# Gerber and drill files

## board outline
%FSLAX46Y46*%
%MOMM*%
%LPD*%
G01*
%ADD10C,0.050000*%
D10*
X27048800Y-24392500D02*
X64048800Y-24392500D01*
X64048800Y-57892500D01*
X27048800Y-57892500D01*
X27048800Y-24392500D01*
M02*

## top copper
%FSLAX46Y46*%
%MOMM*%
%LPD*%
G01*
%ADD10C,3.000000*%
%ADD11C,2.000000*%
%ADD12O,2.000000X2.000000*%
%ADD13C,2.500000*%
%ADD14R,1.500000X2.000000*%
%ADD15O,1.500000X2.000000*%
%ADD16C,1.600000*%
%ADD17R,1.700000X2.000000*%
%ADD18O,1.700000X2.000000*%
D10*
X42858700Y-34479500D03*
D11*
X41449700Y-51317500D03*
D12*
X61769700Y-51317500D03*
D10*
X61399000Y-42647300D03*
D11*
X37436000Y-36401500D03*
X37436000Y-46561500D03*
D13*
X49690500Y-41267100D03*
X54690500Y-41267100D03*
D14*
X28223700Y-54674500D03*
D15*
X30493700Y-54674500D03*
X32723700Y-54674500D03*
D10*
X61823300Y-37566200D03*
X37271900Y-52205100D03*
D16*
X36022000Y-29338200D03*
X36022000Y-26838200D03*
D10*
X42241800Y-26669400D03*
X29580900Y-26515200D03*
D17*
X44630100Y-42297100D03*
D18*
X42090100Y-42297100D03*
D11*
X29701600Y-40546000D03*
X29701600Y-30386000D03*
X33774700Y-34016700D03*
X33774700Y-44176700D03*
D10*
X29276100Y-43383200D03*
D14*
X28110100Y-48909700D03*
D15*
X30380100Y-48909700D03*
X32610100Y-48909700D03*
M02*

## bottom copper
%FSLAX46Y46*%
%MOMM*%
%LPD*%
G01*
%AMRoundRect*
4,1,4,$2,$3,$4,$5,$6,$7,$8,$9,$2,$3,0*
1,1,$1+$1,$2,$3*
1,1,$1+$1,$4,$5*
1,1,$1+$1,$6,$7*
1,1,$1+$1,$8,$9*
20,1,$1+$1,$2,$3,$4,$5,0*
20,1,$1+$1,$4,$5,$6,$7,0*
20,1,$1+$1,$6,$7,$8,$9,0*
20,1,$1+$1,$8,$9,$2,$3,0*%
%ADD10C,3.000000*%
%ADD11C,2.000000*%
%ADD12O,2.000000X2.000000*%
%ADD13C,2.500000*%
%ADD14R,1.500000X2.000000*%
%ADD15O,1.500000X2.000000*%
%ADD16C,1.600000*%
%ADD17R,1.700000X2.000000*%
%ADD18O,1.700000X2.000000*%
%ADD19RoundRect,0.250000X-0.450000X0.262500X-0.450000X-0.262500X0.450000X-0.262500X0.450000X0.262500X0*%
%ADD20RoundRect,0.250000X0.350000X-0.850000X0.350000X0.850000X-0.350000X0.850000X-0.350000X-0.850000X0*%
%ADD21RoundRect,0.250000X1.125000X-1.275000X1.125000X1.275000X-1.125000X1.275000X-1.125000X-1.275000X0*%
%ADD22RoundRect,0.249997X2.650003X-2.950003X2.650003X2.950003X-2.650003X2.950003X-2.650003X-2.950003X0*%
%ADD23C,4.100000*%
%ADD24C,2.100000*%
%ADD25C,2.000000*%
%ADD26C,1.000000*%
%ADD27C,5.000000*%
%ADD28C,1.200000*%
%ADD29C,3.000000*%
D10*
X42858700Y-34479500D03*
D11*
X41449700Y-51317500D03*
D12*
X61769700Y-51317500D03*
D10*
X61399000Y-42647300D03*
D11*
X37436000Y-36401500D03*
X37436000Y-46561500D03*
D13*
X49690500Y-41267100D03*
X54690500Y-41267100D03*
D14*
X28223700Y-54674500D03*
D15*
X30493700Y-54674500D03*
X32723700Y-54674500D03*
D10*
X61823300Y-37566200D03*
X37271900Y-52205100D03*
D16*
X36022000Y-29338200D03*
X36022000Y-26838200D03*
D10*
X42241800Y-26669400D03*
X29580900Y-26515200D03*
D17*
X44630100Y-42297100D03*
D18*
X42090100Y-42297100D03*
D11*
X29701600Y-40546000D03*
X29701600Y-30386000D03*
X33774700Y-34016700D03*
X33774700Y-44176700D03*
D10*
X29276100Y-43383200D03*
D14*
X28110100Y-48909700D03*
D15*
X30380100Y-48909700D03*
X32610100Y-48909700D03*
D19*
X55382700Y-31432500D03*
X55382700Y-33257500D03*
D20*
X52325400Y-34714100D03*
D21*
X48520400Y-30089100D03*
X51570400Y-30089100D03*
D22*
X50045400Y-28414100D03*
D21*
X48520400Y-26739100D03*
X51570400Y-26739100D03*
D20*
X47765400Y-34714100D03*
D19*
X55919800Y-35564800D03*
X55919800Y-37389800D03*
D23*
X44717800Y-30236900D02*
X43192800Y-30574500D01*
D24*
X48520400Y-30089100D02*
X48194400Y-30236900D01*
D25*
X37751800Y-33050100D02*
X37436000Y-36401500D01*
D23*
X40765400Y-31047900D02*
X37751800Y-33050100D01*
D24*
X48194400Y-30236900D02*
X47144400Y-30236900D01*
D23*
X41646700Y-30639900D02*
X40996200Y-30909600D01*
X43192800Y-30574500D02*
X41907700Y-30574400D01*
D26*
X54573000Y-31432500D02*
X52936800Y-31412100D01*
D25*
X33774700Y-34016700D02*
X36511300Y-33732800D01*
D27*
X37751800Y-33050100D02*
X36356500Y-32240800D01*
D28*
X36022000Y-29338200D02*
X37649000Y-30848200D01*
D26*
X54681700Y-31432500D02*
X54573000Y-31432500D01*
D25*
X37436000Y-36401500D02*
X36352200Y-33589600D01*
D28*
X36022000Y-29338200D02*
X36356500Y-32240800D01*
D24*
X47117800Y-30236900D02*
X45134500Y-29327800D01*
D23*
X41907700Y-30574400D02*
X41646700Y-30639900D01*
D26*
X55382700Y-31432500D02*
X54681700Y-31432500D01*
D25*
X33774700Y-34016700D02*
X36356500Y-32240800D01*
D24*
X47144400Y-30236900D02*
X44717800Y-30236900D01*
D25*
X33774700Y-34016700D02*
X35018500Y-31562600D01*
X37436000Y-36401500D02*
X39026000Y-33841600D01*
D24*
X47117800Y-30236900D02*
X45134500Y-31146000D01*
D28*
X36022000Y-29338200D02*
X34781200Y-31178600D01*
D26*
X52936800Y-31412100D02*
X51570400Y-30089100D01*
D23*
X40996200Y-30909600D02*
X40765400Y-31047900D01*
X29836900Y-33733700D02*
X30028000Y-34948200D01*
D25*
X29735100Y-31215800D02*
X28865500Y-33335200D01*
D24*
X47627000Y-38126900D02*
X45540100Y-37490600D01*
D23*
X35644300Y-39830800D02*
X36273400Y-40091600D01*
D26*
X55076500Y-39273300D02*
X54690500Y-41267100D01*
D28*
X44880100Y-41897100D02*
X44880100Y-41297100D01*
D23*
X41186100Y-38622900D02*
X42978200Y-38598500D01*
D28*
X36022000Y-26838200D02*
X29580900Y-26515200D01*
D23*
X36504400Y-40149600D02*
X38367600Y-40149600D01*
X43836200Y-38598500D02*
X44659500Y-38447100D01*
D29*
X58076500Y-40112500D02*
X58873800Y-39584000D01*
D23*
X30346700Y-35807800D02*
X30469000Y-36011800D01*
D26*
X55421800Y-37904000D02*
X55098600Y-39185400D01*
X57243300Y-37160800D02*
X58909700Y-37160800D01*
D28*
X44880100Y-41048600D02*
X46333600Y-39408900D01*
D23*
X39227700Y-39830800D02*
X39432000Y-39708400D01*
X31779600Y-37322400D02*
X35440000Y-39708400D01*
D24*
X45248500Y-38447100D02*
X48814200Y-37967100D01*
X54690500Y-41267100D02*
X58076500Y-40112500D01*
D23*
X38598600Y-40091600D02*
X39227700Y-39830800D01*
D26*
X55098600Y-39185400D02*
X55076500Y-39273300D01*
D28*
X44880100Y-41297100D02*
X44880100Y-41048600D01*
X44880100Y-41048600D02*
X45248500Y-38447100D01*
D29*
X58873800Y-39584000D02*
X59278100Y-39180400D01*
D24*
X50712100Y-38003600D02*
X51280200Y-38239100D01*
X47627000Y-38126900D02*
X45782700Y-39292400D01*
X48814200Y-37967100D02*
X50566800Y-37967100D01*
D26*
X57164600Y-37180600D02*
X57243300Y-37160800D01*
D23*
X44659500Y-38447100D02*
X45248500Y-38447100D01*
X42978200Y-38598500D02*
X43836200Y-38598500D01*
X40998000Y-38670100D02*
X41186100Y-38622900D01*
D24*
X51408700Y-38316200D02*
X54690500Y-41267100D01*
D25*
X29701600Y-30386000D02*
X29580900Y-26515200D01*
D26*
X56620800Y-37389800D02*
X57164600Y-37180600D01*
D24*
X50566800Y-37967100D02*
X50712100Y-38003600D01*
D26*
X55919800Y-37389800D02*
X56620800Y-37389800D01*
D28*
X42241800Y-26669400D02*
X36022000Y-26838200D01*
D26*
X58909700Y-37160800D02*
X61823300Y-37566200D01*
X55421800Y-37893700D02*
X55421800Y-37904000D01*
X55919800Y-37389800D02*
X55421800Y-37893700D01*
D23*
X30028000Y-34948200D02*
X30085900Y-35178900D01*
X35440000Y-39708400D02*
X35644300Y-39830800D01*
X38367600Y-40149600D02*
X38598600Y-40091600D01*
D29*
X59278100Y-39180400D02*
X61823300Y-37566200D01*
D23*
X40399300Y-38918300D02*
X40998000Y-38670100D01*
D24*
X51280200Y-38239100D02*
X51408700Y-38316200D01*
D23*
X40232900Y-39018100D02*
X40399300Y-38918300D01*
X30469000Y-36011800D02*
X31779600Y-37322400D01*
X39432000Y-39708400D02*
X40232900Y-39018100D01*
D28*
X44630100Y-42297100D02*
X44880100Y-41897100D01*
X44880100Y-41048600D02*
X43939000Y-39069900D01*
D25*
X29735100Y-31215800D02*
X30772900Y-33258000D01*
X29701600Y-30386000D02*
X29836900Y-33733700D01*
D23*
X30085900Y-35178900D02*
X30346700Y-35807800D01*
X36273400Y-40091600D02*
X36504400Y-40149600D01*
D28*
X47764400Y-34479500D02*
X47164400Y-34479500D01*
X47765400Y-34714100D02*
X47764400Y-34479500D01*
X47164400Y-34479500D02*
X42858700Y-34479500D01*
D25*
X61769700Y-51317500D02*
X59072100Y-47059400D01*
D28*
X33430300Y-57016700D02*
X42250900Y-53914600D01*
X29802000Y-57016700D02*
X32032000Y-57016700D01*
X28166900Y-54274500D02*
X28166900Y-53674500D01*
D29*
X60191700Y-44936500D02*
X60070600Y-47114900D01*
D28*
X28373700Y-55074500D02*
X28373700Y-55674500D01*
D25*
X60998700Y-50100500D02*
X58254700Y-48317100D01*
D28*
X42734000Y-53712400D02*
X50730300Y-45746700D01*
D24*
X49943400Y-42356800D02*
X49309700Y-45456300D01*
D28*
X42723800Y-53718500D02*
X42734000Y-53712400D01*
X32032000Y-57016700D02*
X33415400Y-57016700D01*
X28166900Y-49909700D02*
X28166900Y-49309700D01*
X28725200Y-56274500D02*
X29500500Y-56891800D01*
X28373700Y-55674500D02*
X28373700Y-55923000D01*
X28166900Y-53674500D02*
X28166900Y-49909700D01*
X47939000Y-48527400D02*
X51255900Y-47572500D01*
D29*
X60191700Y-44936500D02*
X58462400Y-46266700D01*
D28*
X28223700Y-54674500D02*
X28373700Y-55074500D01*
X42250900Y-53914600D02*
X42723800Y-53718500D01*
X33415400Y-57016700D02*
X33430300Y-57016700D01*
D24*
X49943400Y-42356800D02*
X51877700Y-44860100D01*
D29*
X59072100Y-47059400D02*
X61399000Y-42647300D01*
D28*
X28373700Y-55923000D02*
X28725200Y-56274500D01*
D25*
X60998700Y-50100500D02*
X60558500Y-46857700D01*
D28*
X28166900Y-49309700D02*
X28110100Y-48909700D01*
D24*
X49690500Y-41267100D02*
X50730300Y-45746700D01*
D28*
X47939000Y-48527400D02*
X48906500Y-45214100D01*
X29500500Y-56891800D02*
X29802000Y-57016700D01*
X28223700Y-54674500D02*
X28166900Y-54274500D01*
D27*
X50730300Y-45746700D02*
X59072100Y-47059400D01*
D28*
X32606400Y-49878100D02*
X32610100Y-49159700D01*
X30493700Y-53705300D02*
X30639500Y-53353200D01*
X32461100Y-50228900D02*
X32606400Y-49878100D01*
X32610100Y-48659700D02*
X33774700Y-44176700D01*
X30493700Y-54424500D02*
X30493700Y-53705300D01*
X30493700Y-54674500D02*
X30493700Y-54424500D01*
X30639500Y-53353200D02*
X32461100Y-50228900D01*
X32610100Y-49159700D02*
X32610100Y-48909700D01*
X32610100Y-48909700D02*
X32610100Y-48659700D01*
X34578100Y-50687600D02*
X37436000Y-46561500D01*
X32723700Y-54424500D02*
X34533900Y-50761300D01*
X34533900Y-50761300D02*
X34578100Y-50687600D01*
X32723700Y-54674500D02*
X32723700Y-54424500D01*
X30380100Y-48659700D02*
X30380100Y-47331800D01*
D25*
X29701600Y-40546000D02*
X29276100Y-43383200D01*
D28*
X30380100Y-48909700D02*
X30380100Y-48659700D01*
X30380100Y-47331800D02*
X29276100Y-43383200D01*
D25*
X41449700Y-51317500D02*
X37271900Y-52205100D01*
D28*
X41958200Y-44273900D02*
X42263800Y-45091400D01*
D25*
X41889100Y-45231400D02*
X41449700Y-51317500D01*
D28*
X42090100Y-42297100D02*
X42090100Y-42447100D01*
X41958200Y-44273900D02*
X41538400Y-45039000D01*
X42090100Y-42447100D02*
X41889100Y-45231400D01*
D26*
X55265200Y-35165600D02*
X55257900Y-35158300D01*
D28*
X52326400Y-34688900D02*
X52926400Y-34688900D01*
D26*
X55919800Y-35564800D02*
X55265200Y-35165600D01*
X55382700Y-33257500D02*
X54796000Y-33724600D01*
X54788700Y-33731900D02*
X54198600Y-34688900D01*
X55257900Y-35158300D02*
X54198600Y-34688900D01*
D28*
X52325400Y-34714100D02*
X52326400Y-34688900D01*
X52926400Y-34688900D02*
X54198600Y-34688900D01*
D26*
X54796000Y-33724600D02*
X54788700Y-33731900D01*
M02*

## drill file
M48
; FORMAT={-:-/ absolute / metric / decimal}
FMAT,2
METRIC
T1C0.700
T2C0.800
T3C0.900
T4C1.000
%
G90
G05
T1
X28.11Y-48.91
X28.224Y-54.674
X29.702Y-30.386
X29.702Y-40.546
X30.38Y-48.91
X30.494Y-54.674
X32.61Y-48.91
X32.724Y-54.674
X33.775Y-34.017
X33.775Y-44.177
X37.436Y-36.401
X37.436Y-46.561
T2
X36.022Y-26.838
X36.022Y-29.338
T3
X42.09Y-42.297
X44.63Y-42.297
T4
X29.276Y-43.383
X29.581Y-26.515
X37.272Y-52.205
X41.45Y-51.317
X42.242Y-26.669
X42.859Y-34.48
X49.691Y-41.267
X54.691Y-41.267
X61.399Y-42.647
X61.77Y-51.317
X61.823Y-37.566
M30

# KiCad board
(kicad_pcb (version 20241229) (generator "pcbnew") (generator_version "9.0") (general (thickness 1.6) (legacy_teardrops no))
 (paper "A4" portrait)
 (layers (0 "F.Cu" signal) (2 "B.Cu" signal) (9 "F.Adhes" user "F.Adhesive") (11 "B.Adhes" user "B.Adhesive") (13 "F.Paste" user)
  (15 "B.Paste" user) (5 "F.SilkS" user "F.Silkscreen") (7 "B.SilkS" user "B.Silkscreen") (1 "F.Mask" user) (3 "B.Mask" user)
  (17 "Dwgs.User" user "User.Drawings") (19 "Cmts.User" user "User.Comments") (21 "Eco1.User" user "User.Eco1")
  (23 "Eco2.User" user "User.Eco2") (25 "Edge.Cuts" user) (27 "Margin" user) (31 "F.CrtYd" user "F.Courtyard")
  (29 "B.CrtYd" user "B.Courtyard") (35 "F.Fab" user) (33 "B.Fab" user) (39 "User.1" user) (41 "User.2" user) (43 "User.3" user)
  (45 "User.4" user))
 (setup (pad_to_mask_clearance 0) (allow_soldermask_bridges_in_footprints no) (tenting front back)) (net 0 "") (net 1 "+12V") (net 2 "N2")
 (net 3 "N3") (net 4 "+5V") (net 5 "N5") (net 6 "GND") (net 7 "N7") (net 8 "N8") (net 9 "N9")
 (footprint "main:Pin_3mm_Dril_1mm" (layer "F.Cu") (at 42.8587 34.4795)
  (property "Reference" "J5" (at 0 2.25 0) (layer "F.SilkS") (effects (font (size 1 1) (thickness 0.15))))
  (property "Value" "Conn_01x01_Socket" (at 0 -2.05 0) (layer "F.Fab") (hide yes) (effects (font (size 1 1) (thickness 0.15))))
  (pad "1" thru_hole circle (at 0 0) (size 3 3) (drill 1) (layers "*.Cu" "*.Mask") (remove_unused_layers no) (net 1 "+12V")))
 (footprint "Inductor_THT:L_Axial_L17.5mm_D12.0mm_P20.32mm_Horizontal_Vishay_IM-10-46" (layer "F.Cu") (at 41.4497 51.3175)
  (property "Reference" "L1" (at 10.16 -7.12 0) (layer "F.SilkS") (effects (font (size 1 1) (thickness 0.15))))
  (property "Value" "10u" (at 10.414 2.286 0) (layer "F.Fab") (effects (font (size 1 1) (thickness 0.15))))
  (pad "1" thru_hole circle (at 0 0) (size 2 2) (drill 1) (layers "*.Cu" "*.Mask") (remove_unused_layers no) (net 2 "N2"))
  (pad "2" thru_hole oval (at 20.32 0) (size 2 2) (drill 1) (layers "*.Cu" "*.Mask") (remove_unused_layers no) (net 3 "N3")))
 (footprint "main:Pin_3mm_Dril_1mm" (layer "F.Cu") (at 61.399 42.6473)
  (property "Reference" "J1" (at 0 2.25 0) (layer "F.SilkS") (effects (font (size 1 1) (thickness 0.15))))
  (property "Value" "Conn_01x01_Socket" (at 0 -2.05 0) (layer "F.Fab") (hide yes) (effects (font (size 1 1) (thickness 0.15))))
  (pad "1" thru_hole circle (at 0 0) (size 3 3) (drill 1) (layers "*.Cu" "*.Mask") (remove_unused_layers no) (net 3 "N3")))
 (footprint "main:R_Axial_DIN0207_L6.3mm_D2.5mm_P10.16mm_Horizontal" (layer "F.Cu") (at 37.436 36.4015 -90)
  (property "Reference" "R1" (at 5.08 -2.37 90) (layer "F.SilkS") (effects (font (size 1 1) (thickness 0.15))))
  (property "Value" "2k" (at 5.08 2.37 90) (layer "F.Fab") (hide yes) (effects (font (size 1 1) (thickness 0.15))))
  (pad "1" thru_hole circle (at 0 0 270) (size 2 2) (drill 0.7) (layers "*.Cu" "*.Mask") (remove_unused_layers no) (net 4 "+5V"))
  (pad "2" thru_hole circle (at 10.16 0 270) (size 2 2) (drill 0.7) (layers "*.Cu" "*.Mask") (remove_unused_layers no) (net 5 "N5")))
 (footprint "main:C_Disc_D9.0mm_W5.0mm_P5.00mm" (layer "F.Cu") (at 49.6905 41.2671)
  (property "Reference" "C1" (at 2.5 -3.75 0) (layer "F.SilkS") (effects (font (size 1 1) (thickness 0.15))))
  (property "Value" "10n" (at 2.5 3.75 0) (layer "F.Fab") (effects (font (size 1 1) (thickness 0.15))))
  (pad "1" thru_hole circle (at 0 0) (size 2.5 2.5) (drill 1) (layers "*.Cu" "*.Mask") (remove_unused_layers no) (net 3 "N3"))
  (pad "2" thru_hole circle (at 5 0) (size 2.5 2.5) (drill 1) (layers "*.Cu" "*.Mask") (remove_unused_layers no) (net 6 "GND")))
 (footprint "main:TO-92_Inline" (layer "F.Cu") (at 29.2237 54.6745)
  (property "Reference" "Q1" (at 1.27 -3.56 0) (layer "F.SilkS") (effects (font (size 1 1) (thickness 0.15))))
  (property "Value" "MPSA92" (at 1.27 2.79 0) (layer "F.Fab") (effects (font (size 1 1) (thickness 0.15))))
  (pad "1" thru_hole rect (at -1 0) (size 1.5 2) (drill 0.7) (layers "*.Cu" "*.Mask") (remove_unused_layers no) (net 3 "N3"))
  (pad "2" thru_hole oval (at 1.27 0) (size 1.5 2) (drill 0.7) (layers "*.Cu" "*.Mask") (remove_unused_layers no) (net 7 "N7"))
  (pad "3" thru_hole oval (at 3.5 0) (size 1.5 2) (drill 0.7) (layers "*.Cu" "*.Mask") (remove_unused_layers no) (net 5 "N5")))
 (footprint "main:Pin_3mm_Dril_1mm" (layer "F.Cu") (at 61.8233 37.5662)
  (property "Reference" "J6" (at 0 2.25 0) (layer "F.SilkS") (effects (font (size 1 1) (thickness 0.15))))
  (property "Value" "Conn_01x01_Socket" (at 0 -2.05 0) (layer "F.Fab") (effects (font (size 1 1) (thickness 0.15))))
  (pad "1" thru_hole circle (at 0 0) (size 3 3) (drill 1) (layers "*.Cu" "*.Mask") (remove_unused_layers no) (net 6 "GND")))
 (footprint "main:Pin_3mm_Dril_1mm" (layer "F.Cu") (at 37.2719 52.2051)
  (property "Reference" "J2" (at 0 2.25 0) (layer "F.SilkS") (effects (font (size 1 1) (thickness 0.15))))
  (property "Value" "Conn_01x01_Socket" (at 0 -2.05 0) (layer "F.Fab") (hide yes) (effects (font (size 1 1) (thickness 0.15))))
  (pad "1" thru_hole circle (at 0 0) (size 3 3) (drill 1) (layers "*.Cu" "*.Mask") (remove_unused_layers no) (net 2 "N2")))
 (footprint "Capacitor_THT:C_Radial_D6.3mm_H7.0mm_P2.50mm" (layer "F.Cu") (at 36.022 29.3382 90)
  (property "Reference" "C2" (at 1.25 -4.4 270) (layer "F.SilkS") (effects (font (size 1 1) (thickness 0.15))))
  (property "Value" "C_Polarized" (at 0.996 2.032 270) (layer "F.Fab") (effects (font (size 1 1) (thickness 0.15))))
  (pad "1" thru_hole circle (at 0 0 90) (size 1.6 1.6) (drill 0.8) (layers "*.Cu" "*.Mask") (remove_unused_layers no) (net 4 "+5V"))
  (pad "2" thru_hole circle (at 2.5 0 90) (size 1.6 1.6) (drill 0.8) (layers "*.Cu" "*.Mask") (remove_unused_layers no) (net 6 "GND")))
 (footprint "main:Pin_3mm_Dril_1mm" (layer "F.Cu") (at 42.2418 26.6694 -90)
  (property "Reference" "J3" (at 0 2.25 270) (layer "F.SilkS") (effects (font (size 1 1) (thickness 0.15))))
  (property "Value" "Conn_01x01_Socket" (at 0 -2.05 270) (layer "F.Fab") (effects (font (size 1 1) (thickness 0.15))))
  (pad "1" thru_hole circle (at 0 0 270) (size 3 3) (drill 1) (layers "*.Cu" "*.Mask") (remove_unused_layers no) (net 6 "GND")))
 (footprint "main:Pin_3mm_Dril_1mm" (layer "F.Cu") (at 29.5809 26.5152)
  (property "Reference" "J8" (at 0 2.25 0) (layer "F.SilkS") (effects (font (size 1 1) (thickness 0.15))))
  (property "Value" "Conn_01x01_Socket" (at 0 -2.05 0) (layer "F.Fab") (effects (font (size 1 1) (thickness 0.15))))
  (pad "1" thru_hole circle (at 0 0) (size 3 3) (drill 1) (layers "*.Cu" "*.Mask") (remove_unused_layers no) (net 6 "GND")))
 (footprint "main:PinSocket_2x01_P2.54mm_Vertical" (layer "F.Cu") (at 44.6301 42.2971)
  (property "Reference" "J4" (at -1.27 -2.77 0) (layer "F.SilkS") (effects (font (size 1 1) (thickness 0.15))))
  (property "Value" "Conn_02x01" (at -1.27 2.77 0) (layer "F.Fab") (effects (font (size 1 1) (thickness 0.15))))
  (pad "1" thru_hole rect (at 0 0) (size 1.7 2) (drill 0.9) (layers "*.Cu" "*.Mask") (remove_unused_layers no) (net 6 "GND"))
  (pad "2" thru_hole oval (at -2.54 0) (size 1.7 2) (drill 0.9) (layers "*.Cu" "*.Mask") (remove_unused_layers no) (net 2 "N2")))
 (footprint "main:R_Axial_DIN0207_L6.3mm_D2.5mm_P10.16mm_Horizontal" (layer "F.Cu") (at 29.7016 40.546 90)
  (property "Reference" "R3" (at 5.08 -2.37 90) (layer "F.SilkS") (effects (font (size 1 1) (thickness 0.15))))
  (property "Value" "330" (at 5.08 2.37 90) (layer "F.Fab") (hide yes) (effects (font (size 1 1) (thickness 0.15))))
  (pad "1" thru_hole circle (at 0 0 90) (size 2 2) (drill 0.7) (layers "*.Cu" "*.Mask") (remove_unused_layers no) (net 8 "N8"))
  (pad "2" thru_hole circle (at 10.16 0 90) (size 2 2) (drill 0.7) (layers "*.Cu" "*.Mask") (remove_unused_layers no) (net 6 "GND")))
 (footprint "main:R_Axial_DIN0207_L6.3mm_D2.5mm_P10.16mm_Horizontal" (layer "F.Cu") (at 33.7747 34.0167 -90)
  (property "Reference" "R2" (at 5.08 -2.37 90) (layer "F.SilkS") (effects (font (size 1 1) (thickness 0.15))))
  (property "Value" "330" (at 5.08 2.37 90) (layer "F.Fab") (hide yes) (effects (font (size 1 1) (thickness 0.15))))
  (pad "1" thru_hole circle (at 0 0 270) (size 2 2) (drill 0.7) (layers "*.Cu" "*.Mask") (remove_unused_layers no) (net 4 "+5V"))
  (pad "2" thru_hole circle (at 10.16 0 270) (size 2 2) (drill 0.7) (layers "*.Cu" "*.Mask") (remove_unused_layers no) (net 7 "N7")))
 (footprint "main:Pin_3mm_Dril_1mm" (layer "F.Cu") (at 29.2761 43.3832)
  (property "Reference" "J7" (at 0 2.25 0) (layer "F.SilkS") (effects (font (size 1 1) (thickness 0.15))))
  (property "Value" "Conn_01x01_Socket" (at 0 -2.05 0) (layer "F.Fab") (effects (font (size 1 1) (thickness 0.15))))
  (pad "1" thru_hole circle (at 0 0) (size 3 3) (drill 1) (layers "*.Cu" "*.Mask") (remove_unused_layers no) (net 8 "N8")))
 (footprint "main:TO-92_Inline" (layer "F.Cu") (at 29.1101 48.9097)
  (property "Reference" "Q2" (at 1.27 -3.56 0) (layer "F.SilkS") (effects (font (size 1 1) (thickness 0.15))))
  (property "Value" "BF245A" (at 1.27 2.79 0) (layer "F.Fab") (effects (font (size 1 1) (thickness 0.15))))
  (pad "1" thru_hole rect (at -1 0) (size 1.5 2) (drill 0.7) (layers "*.Cu" "*.Mask") (remove_unused_layers no) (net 3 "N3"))
  (pad "2" thru_hole oval (at 1.27 0) (size 1.5 2) (drill 0.7) (layers "*.Cu" "*.Mask") (remove_unused_layers no) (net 8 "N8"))
  (pad "3" thru_hole oval (at 3.5 0) (size 1.5 2) (drill 0.7) (layers "*.Cu" "*.Mask") (remove_unused_layers no) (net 7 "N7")))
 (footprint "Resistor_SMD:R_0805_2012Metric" (layer "B.Cu") (at 55.3827 32.345 -90)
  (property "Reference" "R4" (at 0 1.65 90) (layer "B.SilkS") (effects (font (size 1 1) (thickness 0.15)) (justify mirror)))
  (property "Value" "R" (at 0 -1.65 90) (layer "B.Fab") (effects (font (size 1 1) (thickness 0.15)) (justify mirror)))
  (pad "1" smd roundrect (at -0.9125 0 270) (size 1.025 1.4) (layers "B.Cu" "B.Mask" "B.Paste") (roundrect_rratio 0.243902) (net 4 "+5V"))
  (pad "2" smd roundrect (at 0.9125 0 270) (size 1.025 1.4) (layers "B.Cu" "B.Mask" "B.Paste") (roundrect_rratio 0.243902) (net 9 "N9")))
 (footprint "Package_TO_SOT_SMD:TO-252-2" (layer "B.Cu") (at 50.0454 29.6741 90)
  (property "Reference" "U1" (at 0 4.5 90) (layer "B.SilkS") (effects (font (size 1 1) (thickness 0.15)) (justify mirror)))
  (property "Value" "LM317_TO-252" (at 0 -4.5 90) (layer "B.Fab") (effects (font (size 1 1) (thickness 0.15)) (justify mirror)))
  (pad "1" smd roundrect (at -5.04 2.28 90) (size 2.2 1.2) (layers "B.Cu" "B.Mask" "B.Paste") (roundrect_rratio 0.208333) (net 9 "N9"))
  (pad "2" smd roundrect (at -0.415 -1.525 90) (size 3.05 2.75) (layers "B.Cu" "B.Paste") (roundrect_rratio 0.090909) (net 4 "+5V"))
  (pad "2" smd roundrect (at -0.415 1.525 90) (size 3.05 2.75) (layers "B.Cu" "B.Paste") (roundrect_rratio 0.090909) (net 4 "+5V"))
  (pad "2" smd roundrect (at 1.26 0 90) (size 6.4 5.8) (layers "B.Cu" "B.Mask") (roundrect_rratio 0.043103) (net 4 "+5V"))
  (pad "2" smd roundrect (at 2.935 -1.525 90) (size 3.05 2.75) (layers "B.Cu" "B.Paste") (roundrect_rratio 0.090909) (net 4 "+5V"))
  (pad "2" smd roundrect (at 2.935 1.525 90) (size 3.05 2.75) (layers "B.Cu" "B.Paste") (roundrect_rratio 0.090909) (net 4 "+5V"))
  (pad "3" smd roundrect (at -5.04 -2.28 90) (size 2.2 1.2) (layers "B.Cu" "B.Mask" "B.Paste") (roundrect_rratio 0.208333) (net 1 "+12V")))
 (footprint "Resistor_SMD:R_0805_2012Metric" (layer "B.Cu") (at 55.9198 36.4773 -90)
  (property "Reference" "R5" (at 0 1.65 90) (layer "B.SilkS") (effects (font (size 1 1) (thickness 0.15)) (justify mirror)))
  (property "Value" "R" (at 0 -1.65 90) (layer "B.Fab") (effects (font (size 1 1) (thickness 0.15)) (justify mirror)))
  (pad "1" smd roundrect (at -0.9125 0 270) (size 1.025 1.4) (layers "B.Cu" "B.Mask" "B.Paste") (roundrect_rratio 0.243902) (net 9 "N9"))
  (pad "2" smd roundrect (at 0.9125 0 270) (size 1.025 1.4) (layers "B.Cu" "B.Mask" "B.Paste") (roundrect_rratio 0.243902) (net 6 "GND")))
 (gr_rect (start 27.0488 24.3925) (end 64.0488 57.8925) (stroke (width 0.05) (type default)) (fill no) (layer "Edge.Cuts"))
 (segment (start 44.7178 30.2369) (end 43.1928 30.5745) (width 4.1) (layer "B.Cu") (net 4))
 (segment (start 48.5204 30.0891) (end 48.1944 30.2369) (width 2.1) (layer "B.Cu") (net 4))
 (segment (start 37.7518 33.0501) (end 37.436 36.4015) (width 2) (layer "B.Cu") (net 4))
 (segment (start 40.7654 31.0479) (end 37.7518 33.0501) (width 4.1) (layer "B.Cu") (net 4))
 (segment (start 48.1944 30.2369) (end 47.1444 30.2369) (width 2.1) (layer "B.Cu") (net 4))
 (segment (start 41.6467 30.6399) (end 40.9962 30.9096) (width 4.1) (layer "B.Cu") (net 4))
 (segment (start 43.1928 30.5745) (end 41.9077 30.5744) (width 4.1) (layer "B.Cu") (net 4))
 (segment (start 54.573 31.4325) (end 52.9368 31.4121) (width 1) (layer "B.Cu") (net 4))
 (segment (start 33.7747 34.0167) (end 36.5113 33.7328) (width 2) (layer "B.Cu") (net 4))
 (segment (start 37.7518 33.0501) (end 36.3565 32.2408) (width 5) (layer "B.Cu") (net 4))
 (segment (start 36.022 29.3382) (end 37.649 30.8482) (width 1.2) (layer "B.Cu") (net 4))
 (segment (start 54.6817 31.4325) (end 54.573 31.4325) (width 1) (layer "B.Cu") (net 4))
 (segment (start 37.436 36.4015) (end 36.3522 33.5896) (width 2) (layer "B.Cu") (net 4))
 (segment (start 36.022 29.3382) (end 36.3565 32.2408) (width 1.2) (layer "B.Cu") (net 4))
 (segment (start 47.1178 30.2369) (end 45.1345 29.3278) (width 2.1) (layer "B.Cu") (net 4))
 (segment (start 41.9077 30.5744) (end 41.6467 30.6399) (width 4.1) (layer "B.Cu") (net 4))
 (segment (start 55.3827 31.4325) (end 54.6817 31.4325) (width 1) (layer "B.Cu") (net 4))
 (segment (start 33.7747 34.0167) (end 36.3565 32.2408) (width 2) (layer "B.Cu") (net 4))
 (segment (start 47.1444 30.2369) (end 44.7178 30.2369) (width 2.1) (layer "B.Cu") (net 4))
 (segment (start 33.7747 34.0167) (end 35.0185 31.5626) (width 2) (layer "B.Cu") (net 4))
 (segment (start 37.436 36.4015) (end 39.026 33.8416) (width 2) (layer "B.Cu") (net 4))
 (segment (start 47.1178 30.2369) (end 45.1345 31.146) (width 2.1) (layer "B.Cu") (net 4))
 (segment (start 36.022 29.3382) (end 34.7812 31.1786) (width 1.2) (layer "B.Cu") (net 4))
 (segment (start 52.9368 31.4121) (end 51.5704 30.0891) (width 1) (layer "B.Cu") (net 4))
 (segment (start 40.9962 30.9096) (end 40.7654 31.0479) (width 4.1) (layer "B.Cu") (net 4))
 (segment (start 29.8369 33.7337) (end 30.028 34.9482) (width 4.1) (layer "B.Cu") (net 6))
 (segment (start 29.7351 31.2158) (end 28.8655 33.3352) (width 2) (layer "B.Cu") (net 6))
 (segment (start 47.627 38.1269) (end 45.5401 37.4906) (width 2.1) (layer "B.Cu") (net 6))
 (segment (start 35.6443 39.8308) (end 36.2734 40.0916) (width 4.1) (layer "B.Cu") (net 6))
 (segment (start 55.0765 39.2733) (end 54.6905 41.2671) (width 1) (layer "B.Cu") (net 6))
 (segment (start 44.8801 41.8971) (end 44.8801 41.2971) (width 1.2) (layer "B.Cu") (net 6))
 (segment (start 41.1861 38.6229) (end 42.9782 38.5985) (width 4.1) (layer "B.Cu") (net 6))
 (segment (start 36.022 26.8382) (end 29.5809 26.5152) (width 1.2) (layer "B.Cu") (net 6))
 (segment (start 36.5044 40.1496) (end 38.3676 40.1496) (width 4.1) (layer "B.Cu") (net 6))
 (segment (start 43.8362 38.5985) (end 44.6595 38.4471) (width 4.1) (layer "B.Cu") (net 6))
 (segment (start 58.0765 40.1125) (end 58.8738 39.584) (width 3) (layer "B.Cu") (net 6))
 (segment (start 30.3467 35.8078) (end 30.469 36.0118) (width 4.1) (layer "B.Cu") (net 6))
 (segment (start 55.4218 37.904) (end 55.0986 39.1854) (width 1) (layer "B.Cu") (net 6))
 (segment (start 57.2433 37.1608) (end 58.9097 37.1608) (width 1) (layer "B.Cu") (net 6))
 (segment (start 44.8801 41.0486) (end 46.3336 39.4089) (width 1.2) (layer "B.Cu") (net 6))
 (segment (start 39.2277 39.8308) (end 39.432 39.7084) (width 4.1) (layer "B.Cu") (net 6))
 (segment (start 31.7796 37.3224) (end 35.44 39.7084) (width 4.1) (layer "B.Cu") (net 6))
 (segment (start 45.2485 38.4471) (end 48.8142 37.9671) (width 2.1) (layer "B.Cu") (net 6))
 (segment (start 54.6905 41.2671) (end 58.0765 40.1125) (width 2.1) (layer "B.Cu") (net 6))
 (segment (start 38.5986 40.0916) (end 39.2277 39.8308) (width 4.1) (layer "B.Cu") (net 6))
 (segment (start 55.0986 39.1854) (end 55.0765 39.2733) (width 1) (layer "B.Cu") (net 6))
 (segment (start 44.8801 41.2971) (end 44.8801 41.0486) (width 1.2) (layer "B.Cu") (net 6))
 (segment (start 44.8801 41.0486) (end 45.2485 38.4471) (width 1.2) (layer "B.Cu") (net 6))
 (segment (start 58.8738 39.584) (end 59.2781 39.1804) (width 3) (layer "B.Cu") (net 6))
 (segment (start 50.7121 38.0036) (end 51.2802 38.2391) (width 2.1) (layer "B.Cu") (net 6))
 (segment (start 47.627 38.1269) (end 45.7827 39.2924) (width 2.1) (layer "B.Cu") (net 6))
 (segment (start 48.8142 37.9671) (end 50.5668 37.9671) (width 2.1) (layer "B.Cu") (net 6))
 (segment (start 57.1646 37.1806) (end 57.2433 37.1608) (width 1) (layer "B.Cu") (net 6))
 (segment (start 44.6595 38.4471) (end 45.2485 38.4471) (width 4.1) (layer "B.Cu") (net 6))
 (segment (start 42.9782 38.5985) (end 43.8362 38.5985) (width 4.1) (layer "B.Cu") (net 6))
 (segment (start 40.998 38.6701) (end 41.1861 38.6229) (width 4.1) (layer "B.Cu") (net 6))
 (segment (start 51.4087 38.3162) (end 54.6905 41.2671) (width 2.1) (layer "B.Cu") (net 6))
 (segment (start 29.7016 30.386) (end 29.5809 26.5152) (width 2) (layer "B.Cu") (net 6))
 (segment (start 56.6208 37.3898) (end 57.1646 37.1806) (width 1) (layer "B.Cu") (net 6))
 (segment (start 50.5668 37.9671) (end 50.7121 38.0036) (width 2.1) (layer "B.Cu") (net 6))
 (segment (start 55.9198 37.3898) (end 56.6208 37.3898) (width 1) (layer "B.Cu") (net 6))
 (segment (start 42.2418 26.6694) (end 36.022 26.8382) (width 1.2) (layer "B.Cu") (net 6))
 (segment (start 58.9097 37.1608) (end 61.8233 37.5662) (width 1) (layer "B.Cu") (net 6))
 (segment (start 55.4218 37.8937) (end 55.4218 37.904) (width 1) (layer "B.Cu") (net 6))
 (segment (start 55.9198 37.3898) (end 55.4218 37.8937) (width 1) (layer "B.Cu") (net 6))
 (segment (start 30.028 34.9482) (end 30.0859 35.1789) (width 4.1) (layer "B.Cu") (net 6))
 (segment (start 35.44 39.7084) (end 35.6443 39.8308) (width 4.1) (layer "B.Cu") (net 6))
 (segment (start 38.3676 40.1496) (end 38.5986 40.0916) (width 4.1) (layer "B.Cu") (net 6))
 (segment (start 59.2781 39.1804) (end 61.8233 37.5662) (width 3) (layer "B.Cu") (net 6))
 (segment (start 40.3993 38.9183) (end 40.998 38.6701) (width 4.1) (layer "B.Cu") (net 6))
 (segment (start 51.2802 38.2391) (end 51.4087 38.3162) (width 2.1) (layer "B.Cu") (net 6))
 (segment (start 40.2329 39.0181) (end 40.3993 38.9183) (width 4.1) (layer "B.Cu") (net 6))
 (segment (start 30.469 36.0118) (end 31.7796 37.3224) (width 4.1) (layer "B.Cu") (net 6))
 (segment (start 39.432 39.7084) (end 40.2329 39.0181) (width 4.1) (layer "B.Cu") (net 6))
 (segment (start 44.6301 42.2971) (end 44.8801 41.8971) (width 1.2) (layer "B.Cu") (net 6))
 (segment (start 44.8801 41.0486) (end 43.939 39.0699) (width 1.2) (layer "B.Cu") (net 6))
 (segment (start 29.7351 31.2158) (end 30.7729 33.258) (width 2) (layer "B.Cu") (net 6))
 (segment (start 29.7016 30.386) (end 29.8369 33.7337) (width 2) (layer "B.Cu") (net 6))
 (segment (start 30.0859 35.1789) (end 30.3467 35.8078) (width 4.1) (layer "B.Cu") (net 6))
 (segment (start 36.2734 40.0916) (end 36.5044 40.1496) (width 4.1) (layer "B.Cu") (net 6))
 (segment (start 47.7644 34.4795) (end 47.1644 34.4795) (width 1.2) (layer "B.Cu") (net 1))
 (segment (start 47.7654 34.7141) (end 47.7644 34.4795) (width 1.2) (layer "B.Cu") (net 1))
 (segment (start 47.1644 34.4795) (end 42.8587 34.4795) (width 1.2) (layer "B.Cu") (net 1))
 (segment (start 61.7697 51.3175) (end 59.0721 47.0594) (width 2) (layer "B.Cu") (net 3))
 (segment (start 33.4303 57.0167) (end 42.2509 53.9146) (width 1.2) (layer "B.Cu") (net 3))
 (segment (start 29.802 57.0167) (end 32.032 57.0167) (width 1.2) (layer "B.Cu") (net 3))
 (segment (start 28.1669 54.2745) (end 28.1669 53.6745) (width 1.2) (layer "B.Cu") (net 3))
 (segment (start 60.1917 44.9365) (end 60.0706 47.1149) (width 3) (layer "B.Cu") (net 3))
 (segment (start 28.3737 55.0745) (end 28.3737 55.6745) (width 1.2) (layer "B.Cu") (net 3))
 (segment (start 60.9987 50.1005) (end 58.2547 48.3171) (width 2) (layer "B.Cu") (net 3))
 (segment (start 42.734 53.7124) (end 50.7303 45.7467) (width 1.2) (layer "B.Cu") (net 3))
 (segment (start 49.9434 42.3568) (end 49.3097 45.4563) (width 2.1) (layer "B.Cu") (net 3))
 (segment (start 42.7238 53.7185) (end 42.734 53.7124) (width 1.2) (layer "B.Cu") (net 3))
 (segment (start 32.032 57.0167) (end 33.4154 57.0167) (width 1.2) (layer "B.Cu") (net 3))
 (segment (start 28.1669 49.9097) (end 28.1669 49.3097) (width 1.2) (layer "B.Cu") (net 3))
 (segment (start 28.7252 56.2745) (end 29.5005 56.8918) (width 1.2) (layer "B.Cu") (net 3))
 (segment (start 28.3737 55.6745) (end 28.3737 55.923) (width 1.2) (layer "B.Cu") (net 3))
 (segment (start 28.1669 53.6745) (end 28.1669 49.9097) (width 1.2) (layer "B.Cu") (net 3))
 (segment (start 47.939 48.5274) (end 51.2559 47.5725) (width 1.2) (layer "B.Cu") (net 3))
 (segment (start 60.1917 44.9365) (end 58.4624 46.2667) (width 3) (layer "B.Cu") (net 3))
 (segment (start 28.2237 54.6745) (end 28.3737 55.0745) (width 1.2) (layer "B.Cu") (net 3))
 (segment (start 42.2509 53.9146) (end 42.7238 53.7185) (width 1.2) (layer "B.Cu") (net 3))
 (segment (start 33.4154 57.0167) (end 33.4303 57.0167) (width 1.2) (layer "B.Cu") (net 3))
 (segment (start 49.9434 42.3568) (end 51.8777 44.8601) (width 2.1) (layer "B.Cu") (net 3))
 (segment (start 59.0721 47.0594) (end 61.399 42.6473) (width 3) (layer "B.Cu") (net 3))
 (segment (start 28.3737 55.923) (end 28.7252 56.2745) (width 1.2) (layer "B.Cu") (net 3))
 (segment (start 60.9987 50.1005) (end 60.5585 46.8577) (width 2) (layer "B.Cu") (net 3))
 (segment (start 28.1669 49.3097) (end 28.1101 48.9097) (width 1.2) (layer "B.Cu") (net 3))
 (segment (start 49.6905 41.2671) (end 50.7303 45.7467) (width 2.1) (layer "B.Cu") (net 3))
 (segment (start 47.939 48.5274) (end 48.9065 45.2141) (width 1.2) (layer "B.Cu") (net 3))
 (segment (start 29.5005 56.8918) (end 29.802 57.0167) (width 1.2) (layer "B.Cu") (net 3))
 (segment (start 28.2237 54.6745) (end 28.1669 54.2745) (width 1.2) (layer "B.Cu") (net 3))
 (segment (start 50.7303 45.7467) (end 59.0721 47.0594) (width 5) (layer "B.Cu") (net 3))
 (segment (start 32.6064 49.8781) (end 32.6101 49.1597) (width 1.2) (layer "B.Cu") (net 7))
 (segment (start 30.4937 53.7053) (end 30.6395 53.3532) (width 1.2) (layer "B.Cu") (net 7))
 (segment (start 32.4611 50.2289) (end 32.6064 49.8781) (width 1.2) (layer "B.Cu") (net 7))
 (segment (start 32.6101 48.6597) (end 33.7747 44.1767) (width 1.2) (layer "B.Cu") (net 7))
 (segment (start 30.4937 54.4245) (end 30.4937 53.7053) (width 1.2) (layer "B.Cu") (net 7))
 (segment (start 30.4937 54.6745) (end 30.4937 54.4245) (width 1.2) (layer "B.Cu") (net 7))
 (segment (start 30.6395 53.3532) (end 32.4611 50.2289) (width 1.2) (layer "B.Cu") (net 7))
 (segment (start 32.6101 49.1597) (end 32.6101 48.9097) (width 1.2) (layer "B.Cu") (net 7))
 (segment (start 32.6101 48.9097) (end 32.6101 48.6597) (width 1.2) (layer "B.Cu") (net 7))
 (segment (start 34.5781 50.6876) (end 37.436 46.5615) (width 1.2) (layer "B.Cu") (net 5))
 (segment (start 32.7237 54.4245) (end 34.5339 50.7613) (width 1.2) (layer "B.Cu") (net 5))
 (segment (start 34.5339 50.7613) (end 34.5781 50.6876) (width 1.2) (layer "B.Cu") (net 5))
 (segment (start 32.7237 54.6745) (end 32.7237 54.4245) (width 1.2) (layer "B.Cu") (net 5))
 (segment (start 30.3801 48.6597) (end 30.3801 47.3318) (width 1.2) (layer "B.Cu") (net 8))
 (segment (start 29.7016 40.546) (end 29.2761 43.3832) (width 2) (layer "B.Cu") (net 8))
 (segment (start 30.3801 48.9097) (end 30.3801 48.6597) (width 1.2) (layer "B.Cu") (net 8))
 (segment (start 30.3801 47.3318) (end 29.2761 43.3832) (width 1.2) (layer "B.Cu") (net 8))
 (segment (start 41.4497 51.3175) (end 37.2719 52.2051) (width 2) (layer "B.Cu") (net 2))
 (segment (start 41.9582 44.2739) (end 42.2638 45.0914) (width 1.2) (layer "B.Cu") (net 2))
 (segment (start 41.8891 45.2314) (end 41.4497 51.3175) (width 2) (layer "B.Cu") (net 2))
 (segment (start 42.0901 42.2971) (end 42.0901 42.4471) (width 1.2) (layer "B.Cu") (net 2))
 (segment (start 41.9582 44.2739) (end 41.5384 45.039) (width 1.2) (layer "B.Cu") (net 2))
 (segment (start 42.0901 42.4471) (end 41.8891 45.2314) (width 1.2) (layer "B.Cu") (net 2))
 (segment (start 55.2652 35.1656) (end 55.2579 35.1583) (width 1) (layer "B.Cu") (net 9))
 (segment (start 52.3264 34.6889) (end 52.9264 34.6889) (width 1.2) (layer "B.Cu") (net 9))
 (segment (start 55.9198 35.5648) (end 55.2652 35.1656) (width 1) (layer "B.Cu") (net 9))
 (segment (start 55.3827 33.2575) (end 54.796 33.7246) (width 1) (layer "B.Cu") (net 9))
 (segment (start 54.7887 33.7319) (end 54.1986 34.6889) (width 1) (layer "B.Cu") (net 9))
 (segment (start 55.2579 35.1583) (end 54.1986 34.6889) (width 1) (layer "B.Cu") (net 9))
 (segment (start 52.3254 34.7141) (end 52.3264 34.6889) (width 1.2) (layer "B.Cu") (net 9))
 (segment (start 52.9264 34.6889) (end 54.1986 34.6889) (width 1.2) (layer "B.Cu") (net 9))
 (segment (start 54.796 33.7246) (end 54.7887 33.7319) (width 1) (layer "B.Cu") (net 9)))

